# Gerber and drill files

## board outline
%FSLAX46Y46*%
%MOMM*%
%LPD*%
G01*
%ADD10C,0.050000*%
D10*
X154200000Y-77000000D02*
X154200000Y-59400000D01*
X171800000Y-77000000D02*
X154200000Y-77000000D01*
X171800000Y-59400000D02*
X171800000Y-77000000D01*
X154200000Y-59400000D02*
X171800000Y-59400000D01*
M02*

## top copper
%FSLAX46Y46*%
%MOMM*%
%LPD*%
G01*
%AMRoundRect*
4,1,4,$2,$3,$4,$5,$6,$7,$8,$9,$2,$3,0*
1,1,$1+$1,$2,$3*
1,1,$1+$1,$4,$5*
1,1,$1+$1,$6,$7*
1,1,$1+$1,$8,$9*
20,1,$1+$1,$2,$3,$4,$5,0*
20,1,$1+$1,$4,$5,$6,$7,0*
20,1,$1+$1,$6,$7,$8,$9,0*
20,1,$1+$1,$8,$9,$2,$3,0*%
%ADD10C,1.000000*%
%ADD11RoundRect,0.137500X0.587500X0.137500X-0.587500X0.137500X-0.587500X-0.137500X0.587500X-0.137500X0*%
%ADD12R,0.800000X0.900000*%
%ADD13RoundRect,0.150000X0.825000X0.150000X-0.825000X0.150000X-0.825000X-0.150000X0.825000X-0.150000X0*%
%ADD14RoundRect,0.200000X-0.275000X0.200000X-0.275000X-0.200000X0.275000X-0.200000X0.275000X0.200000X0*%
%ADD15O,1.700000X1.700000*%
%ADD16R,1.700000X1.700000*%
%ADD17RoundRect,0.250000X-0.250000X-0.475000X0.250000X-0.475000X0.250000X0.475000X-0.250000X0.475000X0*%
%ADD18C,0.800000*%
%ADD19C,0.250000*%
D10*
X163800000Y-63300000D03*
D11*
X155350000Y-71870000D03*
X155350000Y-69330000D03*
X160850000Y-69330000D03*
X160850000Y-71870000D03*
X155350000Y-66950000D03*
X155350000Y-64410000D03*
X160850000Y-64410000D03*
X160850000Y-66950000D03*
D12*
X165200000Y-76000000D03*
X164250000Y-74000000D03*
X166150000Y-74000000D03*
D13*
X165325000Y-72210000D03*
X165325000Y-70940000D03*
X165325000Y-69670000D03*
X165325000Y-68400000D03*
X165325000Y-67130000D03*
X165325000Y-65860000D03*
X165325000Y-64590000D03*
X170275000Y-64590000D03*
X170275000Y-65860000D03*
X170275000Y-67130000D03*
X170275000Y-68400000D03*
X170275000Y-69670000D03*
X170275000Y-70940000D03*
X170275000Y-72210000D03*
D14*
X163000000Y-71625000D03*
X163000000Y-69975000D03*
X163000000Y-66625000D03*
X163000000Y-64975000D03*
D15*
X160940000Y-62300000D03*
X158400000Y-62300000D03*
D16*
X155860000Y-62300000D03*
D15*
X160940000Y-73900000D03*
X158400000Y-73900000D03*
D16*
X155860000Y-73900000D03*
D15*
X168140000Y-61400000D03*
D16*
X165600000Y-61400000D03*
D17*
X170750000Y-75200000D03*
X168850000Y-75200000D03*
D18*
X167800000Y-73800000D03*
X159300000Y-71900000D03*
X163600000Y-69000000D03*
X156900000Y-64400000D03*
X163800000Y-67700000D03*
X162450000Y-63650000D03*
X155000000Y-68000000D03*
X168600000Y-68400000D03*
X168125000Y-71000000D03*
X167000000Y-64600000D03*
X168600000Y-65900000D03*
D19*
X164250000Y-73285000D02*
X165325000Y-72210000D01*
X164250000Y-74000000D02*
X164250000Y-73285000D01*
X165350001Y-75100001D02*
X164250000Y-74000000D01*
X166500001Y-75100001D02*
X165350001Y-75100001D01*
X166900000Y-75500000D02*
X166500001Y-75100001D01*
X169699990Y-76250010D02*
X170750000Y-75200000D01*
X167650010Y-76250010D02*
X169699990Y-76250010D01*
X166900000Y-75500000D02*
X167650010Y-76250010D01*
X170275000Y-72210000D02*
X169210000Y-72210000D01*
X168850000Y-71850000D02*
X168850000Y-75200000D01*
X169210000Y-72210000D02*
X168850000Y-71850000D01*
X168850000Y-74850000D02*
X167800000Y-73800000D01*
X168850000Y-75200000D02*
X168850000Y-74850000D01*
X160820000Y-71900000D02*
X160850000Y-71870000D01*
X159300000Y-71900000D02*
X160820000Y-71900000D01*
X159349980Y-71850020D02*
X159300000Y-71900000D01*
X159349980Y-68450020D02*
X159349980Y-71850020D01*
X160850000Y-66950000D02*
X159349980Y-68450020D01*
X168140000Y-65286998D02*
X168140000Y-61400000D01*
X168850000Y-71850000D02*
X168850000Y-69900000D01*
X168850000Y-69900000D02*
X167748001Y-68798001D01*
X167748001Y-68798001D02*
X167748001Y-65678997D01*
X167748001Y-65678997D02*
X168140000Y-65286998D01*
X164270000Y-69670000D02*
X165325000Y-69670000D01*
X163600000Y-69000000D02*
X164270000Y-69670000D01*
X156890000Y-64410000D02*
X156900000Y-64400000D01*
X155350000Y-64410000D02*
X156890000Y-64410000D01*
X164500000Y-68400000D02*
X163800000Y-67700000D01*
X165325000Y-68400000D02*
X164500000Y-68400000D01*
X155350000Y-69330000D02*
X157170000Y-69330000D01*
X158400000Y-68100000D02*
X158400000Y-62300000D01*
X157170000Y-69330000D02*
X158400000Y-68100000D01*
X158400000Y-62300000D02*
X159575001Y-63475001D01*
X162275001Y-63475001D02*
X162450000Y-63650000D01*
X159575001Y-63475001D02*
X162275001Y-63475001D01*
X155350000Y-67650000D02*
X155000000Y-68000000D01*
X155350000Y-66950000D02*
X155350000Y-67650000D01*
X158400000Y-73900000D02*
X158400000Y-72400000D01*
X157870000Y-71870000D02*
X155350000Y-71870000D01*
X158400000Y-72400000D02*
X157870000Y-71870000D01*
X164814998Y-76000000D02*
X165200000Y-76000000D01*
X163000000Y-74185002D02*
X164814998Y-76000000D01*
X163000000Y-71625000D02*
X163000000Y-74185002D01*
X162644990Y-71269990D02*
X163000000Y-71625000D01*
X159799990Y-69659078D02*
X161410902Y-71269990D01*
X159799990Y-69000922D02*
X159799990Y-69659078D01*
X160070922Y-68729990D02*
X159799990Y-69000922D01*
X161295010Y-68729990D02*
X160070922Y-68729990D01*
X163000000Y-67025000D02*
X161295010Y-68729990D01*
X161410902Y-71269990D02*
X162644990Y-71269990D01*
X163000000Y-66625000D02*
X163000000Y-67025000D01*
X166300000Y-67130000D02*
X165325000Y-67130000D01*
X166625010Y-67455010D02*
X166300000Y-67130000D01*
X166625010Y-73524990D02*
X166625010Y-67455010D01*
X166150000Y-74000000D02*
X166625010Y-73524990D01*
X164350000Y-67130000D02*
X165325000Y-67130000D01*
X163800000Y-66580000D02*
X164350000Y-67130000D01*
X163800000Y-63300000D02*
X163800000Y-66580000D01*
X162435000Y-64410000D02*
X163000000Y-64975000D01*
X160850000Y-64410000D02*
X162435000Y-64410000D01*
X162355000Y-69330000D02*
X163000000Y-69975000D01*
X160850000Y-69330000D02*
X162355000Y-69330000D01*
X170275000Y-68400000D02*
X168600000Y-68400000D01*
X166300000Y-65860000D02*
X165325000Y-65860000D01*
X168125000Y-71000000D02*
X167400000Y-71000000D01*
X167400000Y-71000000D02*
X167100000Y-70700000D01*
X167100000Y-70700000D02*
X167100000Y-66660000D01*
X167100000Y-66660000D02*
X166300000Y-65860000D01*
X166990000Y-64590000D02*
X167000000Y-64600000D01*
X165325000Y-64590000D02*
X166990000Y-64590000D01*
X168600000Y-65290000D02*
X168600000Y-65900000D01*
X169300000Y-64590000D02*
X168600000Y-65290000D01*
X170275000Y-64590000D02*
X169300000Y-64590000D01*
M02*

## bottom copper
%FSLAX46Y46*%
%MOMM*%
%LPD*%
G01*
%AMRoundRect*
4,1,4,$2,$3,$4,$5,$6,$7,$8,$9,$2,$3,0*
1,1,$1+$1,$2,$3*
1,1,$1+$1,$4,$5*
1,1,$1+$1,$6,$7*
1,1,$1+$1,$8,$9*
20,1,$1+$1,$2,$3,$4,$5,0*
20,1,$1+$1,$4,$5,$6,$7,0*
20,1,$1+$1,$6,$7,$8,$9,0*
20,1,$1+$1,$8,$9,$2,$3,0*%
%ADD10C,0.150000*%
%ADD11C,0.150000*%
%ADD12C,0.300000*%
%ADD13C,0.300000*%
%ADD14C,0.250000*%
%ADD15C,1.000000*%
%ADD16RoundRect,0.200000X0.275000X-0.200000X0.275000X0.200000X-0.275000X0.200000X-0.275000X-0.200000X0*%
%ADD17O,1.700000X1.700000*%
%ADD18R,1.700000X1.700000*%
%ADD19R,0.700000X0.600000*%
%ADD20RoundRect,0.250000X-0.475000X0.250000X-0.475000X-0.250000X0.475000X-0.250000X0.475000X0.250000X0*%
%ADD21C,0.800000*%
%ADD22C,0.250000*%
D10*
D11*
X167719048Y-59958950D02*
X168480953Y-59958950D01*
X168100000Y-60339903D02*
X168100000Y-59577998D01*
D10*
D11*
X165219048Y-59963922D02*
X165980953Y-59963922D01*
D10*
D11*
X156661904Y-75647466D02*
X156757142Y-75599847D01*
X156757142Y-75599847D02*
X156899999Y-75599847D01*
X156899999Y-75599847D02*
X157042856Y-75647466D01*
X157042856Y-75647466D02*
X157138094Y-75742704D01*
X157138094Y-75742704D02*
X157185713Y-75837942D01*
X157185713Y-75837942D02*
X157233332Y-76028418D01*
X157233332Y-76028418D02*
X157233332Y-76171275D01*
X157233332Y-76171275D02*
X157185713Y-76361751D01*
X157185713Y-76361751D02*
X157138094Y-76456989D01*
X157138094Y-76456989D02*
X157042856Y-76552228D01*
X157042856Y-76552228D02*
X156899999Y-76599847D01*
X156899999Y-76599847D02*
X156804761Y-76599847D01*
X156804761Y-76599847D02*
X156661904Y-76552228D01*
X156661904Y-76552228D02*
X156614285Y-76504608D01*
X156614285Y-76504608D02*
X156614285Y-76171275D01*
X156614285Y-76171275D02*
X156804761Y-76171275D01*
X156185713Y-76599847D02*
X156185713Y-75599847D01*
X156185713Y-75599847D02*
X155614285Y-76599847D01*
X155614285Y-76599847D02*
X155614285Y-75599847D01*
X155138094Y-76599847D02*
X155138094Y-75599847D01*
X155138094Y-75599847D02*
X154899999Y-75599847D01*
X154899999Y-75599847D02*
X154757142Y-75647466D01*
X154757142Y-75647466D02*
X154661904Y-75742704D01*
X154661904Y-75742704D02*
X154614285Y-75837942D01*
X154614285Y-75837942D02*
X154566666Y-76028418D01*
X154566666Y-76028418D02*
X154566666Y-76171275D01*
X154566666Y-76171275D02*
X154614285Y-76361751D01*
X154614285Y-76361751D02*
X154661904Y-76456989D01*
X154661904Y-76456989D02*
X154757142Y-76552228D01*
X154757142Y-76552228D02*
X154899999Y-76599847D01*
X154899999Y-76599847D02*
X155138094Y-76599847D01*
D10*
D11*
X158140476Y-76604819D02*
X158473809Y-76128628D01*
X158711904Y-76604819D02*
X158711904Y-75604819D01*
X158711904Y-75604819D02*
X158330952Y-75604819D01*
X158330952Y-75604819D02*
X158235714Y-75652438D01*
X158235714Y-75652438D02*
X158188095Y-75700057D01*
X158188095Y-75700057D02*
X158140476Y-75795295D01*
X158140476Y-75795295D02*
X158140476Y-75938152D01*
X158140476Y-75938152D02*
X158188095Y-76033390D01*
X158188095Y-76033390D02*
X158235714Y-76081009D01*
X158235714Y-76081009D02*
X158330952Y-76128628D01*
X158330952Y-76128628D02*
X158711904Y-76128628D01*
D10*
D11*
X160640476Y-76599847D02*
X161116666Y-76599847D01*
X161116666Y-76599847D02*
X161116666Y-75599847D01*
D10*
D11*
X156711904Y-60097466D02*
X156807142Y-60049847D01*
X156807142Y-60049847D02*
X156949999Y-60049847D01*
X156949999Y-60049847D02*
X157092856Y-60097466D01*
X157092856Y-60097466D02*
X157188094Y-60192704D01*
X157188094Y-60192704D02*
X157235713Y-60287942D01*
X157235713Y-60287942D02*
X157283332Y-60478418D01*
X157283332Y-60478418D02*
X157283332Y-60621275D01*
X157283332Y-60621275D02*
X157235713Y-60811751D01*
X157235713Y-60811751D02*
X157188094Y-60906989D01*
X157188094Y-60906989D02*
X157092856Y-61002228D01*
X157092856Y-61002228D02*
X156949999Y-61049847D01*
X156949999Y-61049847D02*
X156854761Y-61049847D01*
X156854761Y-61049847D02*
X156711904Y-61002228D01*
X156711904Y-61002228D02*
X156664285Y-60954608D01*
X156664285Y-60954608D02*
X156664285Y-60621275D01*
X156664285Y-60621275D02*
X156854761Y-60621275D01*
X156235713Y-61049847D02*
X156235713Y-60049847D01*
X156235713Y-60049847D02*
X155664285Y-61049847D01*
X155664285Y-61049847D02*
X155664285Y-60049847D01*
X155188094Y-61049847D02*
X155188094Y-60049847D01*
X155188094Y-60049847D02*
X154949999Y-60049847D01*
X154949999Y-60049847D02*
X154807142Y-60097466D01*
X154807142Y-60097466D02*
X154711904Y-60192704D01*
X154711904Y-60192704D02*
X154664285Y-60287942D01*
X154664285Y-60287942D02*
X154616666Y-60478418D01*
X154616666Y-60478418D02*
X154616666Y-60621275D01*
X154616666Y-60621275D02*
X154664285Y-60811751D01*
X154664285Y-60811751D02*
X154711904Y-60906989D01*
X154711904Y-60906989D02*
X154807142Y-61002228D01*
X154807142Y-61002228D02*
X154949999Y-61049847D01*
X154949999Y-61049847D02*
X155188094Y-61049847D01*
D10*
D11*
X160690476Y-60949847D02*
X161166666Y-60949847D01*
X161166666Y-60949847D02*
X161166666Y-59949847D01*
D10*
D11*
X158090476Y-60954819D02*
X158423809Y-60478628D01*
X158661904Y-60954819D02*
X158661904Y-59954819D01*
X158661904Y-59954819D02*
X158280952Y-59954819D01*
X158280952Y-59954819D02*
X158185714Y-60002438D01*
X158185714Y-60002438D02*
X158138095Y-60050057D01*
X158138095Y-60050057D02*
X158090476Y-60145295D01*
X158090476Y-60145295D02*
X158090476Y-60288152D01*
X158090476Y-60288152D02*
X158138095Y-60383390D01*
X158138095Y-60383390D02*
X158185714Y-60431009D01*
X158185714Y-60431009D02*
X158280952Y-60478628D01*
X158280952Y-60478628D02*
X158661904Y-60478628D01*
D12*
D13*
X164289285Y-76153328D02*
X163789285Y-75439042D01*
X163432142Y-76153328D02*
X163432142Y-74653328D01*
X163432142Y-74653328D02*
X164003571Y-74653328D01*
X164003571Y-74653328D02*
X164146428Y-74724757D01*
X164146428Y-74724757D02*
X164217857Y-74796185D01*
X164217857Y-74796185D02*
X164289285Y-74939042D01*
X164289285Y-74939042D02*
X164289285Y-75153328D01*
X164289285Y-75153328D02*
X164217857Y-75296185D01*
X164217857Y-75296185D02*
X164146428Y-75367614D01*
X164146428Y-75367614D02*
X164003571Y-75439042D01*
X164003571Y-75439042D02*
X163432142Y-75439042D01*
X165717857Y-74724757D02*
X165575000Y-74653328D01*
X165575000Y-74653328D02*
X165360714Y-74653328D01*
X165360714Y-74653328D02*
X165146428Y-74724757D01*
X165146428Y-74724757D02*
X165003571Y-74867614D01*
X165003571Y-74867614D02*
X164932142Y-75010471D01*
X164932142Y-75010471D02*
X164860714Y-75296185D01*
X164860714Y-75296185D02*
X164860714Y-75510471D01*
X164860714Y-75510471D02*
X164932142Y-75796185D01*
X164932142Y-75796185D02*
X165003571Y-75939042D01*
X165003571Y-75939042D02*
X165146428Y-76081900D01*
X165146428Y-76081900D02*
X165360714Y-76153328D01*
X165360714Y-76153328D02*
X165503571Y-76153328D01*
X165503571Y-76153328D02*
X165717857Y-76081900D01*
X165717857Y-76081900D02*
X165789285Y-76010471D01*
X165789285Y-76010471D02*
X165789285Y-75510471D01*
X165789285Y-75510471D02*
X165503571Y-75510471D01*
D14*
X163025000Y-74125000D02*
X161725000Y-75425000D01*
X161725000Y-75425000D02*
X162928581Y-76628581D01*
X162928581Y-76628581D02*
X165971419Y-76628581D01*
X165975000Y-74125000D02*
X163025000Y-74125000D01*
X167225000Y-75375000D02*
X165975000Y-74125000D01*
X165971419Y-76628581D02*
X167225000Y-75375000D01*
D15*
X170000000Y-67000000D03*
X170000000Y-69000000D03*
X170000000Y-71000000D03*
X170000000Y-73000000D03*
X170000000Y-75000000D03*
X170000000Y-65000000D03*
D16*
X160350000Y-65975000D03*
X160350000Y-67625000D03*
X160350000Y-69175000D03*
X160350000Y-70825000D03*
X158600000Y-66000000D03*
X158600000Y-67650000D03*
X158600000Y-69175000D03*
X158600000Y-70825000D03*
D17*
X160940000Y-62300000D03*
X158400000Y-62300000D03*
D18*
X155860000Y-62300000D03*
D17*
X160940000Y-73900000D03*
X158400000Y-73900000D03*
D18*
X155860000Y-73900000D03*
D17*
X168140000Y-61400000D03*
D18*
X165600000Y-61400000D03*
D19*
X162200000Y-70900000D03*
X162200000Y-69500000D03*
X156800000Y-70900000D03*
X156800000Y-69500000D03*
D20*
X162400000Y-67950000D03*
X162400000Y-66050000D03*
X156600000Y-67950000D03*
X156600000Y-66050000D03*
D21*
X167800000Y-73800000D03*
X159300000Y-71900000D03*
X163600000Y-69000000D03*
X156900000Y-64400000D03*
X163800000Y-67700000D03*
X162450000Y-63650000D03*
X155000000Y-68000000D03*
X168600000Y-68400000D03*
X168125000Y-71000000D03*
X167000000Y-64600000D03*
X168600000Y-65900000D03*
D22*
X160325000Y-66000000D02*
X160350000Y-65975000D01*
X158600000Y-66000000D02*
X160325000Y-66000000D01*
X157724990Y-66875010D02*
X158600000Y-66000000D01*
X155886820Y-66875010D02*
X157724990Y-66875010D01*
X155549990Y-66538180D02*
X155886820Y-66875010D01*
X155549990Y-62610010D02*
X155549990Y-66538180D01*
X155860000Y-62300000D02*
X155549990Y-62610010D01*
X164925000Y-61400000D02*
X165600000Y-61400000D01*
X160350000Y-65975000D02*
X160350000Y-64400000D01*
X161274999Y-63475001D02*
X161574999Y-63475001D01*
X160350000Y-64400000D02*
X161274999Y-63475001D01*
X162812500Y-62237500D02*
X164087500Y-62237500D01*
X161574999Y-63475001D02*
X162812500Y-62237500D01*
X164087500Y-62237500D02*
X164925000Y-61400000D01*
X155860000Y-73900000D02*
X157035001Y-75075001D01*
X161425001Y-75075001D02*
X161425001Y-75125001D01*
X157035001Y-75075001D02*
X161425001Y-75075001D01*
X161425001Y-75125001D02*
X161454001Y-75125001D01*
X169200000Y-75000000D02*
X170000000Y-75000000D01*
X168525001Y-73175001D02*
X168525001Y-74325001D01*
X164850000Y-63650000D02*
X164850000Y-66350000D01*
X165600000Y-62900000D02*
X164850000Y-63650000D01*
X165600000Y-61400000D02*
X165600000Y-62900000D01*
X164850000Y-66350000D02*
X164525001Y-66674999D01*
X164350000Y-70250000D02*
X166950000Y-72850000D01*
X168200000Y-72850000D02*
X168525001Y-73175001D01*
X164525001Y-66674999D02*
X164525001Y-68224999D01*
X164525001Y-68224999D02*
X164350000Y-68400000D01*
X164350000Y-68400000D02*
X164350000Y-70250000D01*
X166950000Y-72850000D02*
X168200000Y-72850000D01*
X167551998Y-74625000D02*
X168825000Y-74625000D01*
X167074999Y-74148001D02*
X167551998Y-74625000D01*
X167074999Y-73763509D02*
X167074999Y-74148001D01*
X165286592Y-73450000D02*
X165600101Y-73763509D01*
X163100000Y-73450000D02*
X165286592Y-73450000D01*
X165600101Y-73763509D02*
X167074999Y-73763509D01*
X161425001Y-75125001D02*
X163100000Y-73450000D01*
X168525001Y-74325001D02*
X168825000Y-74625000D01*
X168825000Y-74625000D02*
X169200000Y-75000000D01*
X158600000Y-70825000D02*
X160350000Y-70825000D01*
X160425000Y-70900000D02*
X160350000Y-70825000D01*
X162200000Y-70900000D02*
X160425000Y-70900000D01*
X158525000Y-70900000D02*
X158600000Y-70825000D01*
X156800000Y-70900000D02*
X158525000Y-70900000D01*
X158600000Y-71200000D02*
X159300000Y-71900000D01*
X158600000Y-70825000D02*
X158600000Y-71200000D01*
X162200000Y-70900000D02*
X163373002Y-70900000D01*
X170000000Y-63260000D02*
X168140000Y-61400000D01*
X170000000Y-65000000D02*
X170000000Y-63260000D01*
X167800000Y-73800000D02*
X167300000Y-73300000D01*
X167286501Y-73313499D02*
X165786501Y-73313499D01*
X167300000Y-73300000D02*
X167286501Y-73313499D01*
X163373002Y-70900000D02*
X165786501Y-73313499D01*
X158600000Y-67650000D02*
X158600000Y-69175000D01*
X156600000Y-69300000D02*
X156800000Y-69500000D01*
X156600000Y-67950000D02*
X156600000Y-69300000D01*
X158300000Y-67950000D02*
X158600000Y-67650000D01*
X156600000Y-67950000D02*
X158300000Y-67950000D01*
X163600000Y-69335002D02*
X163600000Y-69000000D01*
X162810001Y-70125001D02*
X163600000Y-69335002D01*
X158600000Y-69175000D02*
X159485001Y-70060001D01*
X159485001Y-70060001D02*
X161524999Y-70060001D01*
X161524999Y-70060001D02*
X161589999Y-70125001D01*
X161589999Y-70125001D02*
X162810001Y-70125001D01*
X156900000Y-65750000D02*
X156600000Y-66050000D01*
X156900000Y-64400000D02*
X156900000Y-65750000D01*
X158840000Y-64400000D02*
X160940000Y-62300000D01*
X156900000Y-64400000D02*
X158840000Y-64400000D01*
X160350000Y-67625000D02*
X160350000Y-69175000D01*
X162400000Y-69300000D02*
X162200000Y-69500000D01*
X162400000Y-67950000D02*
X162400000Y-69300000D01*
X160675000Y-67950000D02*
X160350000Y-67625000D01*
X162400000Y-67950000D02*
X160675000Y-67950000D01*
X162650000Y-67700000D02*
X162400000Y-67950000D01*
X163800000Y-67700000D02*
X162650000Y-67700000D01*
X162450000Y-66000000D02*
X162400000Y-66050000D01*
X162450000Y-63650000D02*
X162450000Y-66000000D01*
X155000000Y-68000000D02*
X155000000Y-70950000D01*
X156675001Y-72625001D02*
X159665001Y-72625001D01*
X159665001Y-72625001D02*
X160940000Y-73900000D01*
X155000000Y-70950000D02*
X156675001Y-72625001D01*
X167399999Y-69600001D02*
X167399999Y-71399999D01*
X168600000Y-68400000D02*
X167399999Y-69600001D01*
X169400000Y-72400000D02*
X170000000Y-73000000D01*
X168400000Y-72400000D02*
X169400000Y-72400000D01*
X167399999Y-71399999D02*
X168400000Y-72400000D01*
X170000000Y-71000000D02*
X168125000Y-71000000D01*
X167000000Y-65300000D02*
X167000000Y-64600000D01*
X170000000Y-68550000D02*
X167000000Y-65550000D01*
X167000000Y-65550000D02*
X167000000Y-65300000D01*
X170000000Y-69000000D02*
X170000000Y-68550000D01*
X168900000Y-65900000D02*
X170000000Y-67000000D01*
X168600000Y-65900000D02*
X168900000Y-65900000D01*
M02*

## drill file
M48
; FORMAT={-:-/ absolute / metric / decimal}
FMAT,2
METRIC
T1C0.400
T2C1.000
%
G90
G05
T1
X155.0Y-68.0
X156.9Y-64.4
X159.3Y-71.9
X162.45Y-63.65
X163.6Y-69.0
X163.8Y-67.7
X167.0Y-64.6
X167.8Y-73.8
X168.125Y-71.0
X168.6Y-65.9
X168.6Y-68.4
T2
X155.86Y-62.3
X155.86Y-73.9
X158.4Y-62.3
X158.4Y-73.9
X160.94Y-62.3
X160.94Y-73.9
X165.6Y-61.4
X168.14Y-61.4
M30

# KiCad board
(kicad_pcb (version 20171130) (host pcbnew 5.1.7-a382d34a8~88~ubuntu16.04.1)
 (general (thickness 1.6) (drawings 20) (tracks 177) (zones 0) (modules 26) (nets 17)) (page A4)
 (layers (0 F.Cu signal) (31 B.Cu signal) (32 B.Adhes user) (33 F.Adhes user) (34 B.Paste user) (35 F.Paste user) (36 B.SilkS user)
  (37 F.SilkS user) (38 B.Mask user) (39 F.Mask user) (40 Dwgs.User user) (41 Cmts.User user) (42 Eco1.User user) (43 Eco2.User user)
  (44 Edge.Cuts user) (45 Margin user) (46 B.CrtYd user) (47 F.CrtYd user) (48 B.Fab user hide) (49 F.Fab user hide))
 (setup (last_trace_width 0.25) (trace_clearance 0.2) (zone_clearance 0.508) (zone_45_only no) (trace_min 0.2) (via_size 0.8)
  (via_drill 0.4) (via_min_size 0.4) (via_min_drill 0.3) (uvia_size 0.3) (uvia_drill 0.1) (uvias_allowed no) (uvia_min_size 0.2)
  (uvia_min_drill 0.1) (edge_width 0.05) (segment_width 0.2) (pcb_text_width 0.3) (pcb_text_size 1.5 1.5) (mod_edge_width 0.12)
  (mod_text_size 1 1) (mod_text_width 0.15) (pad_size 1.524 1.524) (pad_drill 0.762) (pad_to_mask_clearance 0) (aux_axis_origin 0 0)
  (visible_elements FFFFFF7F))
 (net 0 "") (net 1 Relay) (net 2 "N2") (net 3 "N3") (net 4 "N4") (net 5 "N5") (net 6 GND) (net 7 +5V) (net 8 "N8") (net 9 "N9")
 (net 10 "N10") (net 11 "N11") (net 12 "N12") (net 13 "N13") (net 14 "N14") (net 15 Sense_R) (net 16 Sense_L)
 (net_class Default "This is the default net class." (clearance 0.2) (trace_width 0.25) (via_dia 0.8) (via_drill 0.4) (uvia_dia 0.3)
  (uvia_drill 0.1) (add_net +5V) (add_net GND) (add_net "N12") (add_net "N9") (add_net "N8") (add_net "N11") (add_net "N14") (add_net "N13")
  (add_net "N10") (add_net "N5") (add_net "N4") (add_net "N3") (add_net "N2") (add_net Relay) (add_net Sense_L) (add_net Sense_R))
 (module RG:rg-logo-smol (layer F.Cu) (at 164.55 75.4)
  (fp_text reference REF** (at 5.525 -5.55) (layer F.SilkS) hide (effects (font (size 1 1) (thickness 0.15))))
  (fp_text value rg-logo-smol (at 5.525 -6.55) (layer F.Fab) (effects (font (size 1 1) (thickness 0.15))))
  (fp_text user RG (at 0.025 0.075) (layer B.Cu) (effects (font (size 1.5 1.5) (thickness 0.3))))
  (fp_line (start -1.525 -1.275) (end -2.825 0.025) (layer B.Cu) (width 0.25))
  (fp_line (start -2.825 0.025) (end -1.621419 1.228581) (layer B.Cu) (width 0.25))
  (fp_line (start -1.621419 1.228581) (end 1.421419 1.228581) (layer B.Cu) (width 0.25))
  (fp_line (start 1.425 -1.275) (end -1.525 -1.275) (layer B.Cu) (width 0.25))
  (fp_line (start 2.675 -0.025) (end 1.425 -1.275) (layer B.Cu) (width 0.25))
  (fp_line (start 1.421419 1.228581) (end 2.675 -0.025) (layer B.Cu) (width 0.25)))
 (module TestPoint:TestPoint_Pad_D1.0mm (layer F.Cu) (at 163.8 63.3)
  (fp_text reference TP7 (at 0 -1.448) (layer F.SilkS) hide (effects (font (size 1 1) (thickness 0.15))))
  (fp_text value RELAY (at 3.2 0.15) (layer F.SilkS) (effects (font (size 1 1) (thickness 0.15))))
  (pad 1 smd circle (at 0 0) (size 1 1) (layers F.Cu F.Mask) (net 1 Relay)))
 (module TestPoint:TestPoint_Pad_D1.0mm (layer B.Cu) (at 170 67)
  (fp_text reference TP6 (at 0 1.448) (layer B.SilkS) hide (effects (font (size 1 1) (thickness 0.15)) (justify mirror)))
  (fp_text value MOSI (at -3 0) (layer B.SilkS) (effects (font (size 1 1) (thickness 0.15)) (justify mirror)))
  (pad 1 smd circle (at 0 0) (size 1 1) (layers B.Cu B.Mask) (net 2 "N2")))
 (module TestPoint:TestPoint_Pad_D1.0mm (layer B.Cu) (at 170 69)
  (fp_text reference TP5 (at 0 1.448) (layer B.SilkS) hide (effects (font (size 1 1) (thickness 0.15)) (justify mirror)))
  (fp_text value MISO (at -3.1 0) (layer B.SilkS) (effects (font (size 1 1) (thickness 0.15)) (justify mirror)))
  (pad 1 smd circle (at 0 0) (size 1 1) (layers B.Cu B.Mask) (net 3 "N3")))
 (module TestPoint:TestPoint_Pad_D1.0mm (layer B.Cu) (at 170 71)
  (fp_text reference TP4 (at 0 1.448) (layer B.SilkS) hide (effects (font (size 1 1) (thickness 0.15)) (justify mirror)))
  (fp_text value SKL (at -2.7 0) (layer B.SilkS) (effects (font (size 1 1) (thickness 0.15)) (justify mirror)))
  (pad 1 smd circle (at 0 0) (size 1 1) (layers B.Cu B.Mask) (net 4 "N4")))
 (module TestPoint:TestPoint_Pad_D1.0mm (layer B.Cu) (at 170 73)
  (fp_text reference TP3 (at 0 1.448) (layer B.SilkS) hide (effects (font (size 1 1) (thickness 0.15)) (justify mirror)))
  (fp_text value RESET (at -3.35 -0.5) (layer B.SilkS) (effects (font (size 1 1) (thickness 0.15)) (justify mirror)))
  (pad 1 smd circle (at 0 0) (size 1 1) (layers B.Cu B.Mask) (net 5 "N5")))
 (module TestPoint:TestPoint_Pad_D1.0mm (layer B.Cu) (at 170 75)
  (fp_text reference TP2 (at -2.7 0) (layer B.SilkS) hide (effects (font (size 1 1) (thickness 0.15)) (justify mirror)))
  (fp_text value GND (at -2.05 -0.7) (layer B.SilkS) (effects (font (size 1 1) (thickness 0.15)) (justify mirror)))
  (pad 1 smd circle (at 0 0) (size 1 1) (layers B.Cu B.Mask) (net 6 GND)))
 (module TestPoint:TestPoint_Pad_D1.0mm (layer B.Cu) (at 170 65)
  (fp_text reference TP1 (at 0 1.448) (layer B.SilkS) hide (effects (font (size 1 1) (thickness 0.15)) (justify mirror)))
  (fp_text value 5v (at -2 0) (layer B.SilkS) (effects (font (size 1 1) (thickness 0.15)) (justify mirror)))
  (pad 1 smd circle (at 0 0) (size 1 1) (layers B.Cu B.Mask) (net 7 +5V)))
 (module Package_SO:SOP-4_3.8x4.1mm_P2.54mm (layer F.Cu) (at 158.1 70.6 180)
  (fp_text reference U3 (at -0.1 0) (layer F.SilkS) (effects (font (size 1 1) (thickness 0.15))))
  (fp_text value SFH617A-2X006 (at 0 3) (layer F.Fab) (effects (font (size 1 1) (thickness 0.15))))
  (pad 4 smd roundrect (at 2.75 -1.27 180) (size 1.45 0.55) (layers F.Cu F.Paste F.Mask) (roundrect_rratio 0.25) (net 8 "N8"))
  (pad 3 smd roundrect (at 2.75 1.27 180) (size 1.45 0.55) (layers F.Cu F.Paste F.Mask) (roundrect_rratio 0.25) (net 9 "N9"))
  (pad 2 smd roundrect (at -2.75 1.27 180) (size 1.45 0.55) (layers F.Cu F.Paste F.Mask) (roundrect_rratio 0.25) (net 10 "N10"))
  (pad 1 smd roundrect (at -2.75 -1.27 180) (size 1.45 0.55) (layers F.Cu F.Paste F.Mask) (roundrect_rratio 0.25) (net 7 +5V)))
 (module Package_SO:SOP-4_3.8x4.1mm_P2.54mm (layer F.Cu) (at 158.1 65.68 180)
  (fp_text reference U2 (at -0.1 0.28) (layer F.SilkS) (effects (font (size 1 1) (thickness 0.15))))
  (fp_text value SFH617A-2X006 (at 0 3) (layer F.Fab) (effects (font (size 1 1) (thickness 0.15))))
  (pad 4 smd roundrect (at 2.75 -1.27 180) (size 1.45 0.55) (layers F.Cu F.Paste F.Mask) (roundrect_rratio 0.25) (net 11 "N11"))
  (pad 3 smd roundrect (at 2.75 1.27 180) (size 1.45 0.55) (layers F.Cu F.Paste F.Mask) (roundrect_rratio 0.25) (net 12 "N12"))
  (pad 2 smd roundrect (at -2.75 1.27 180) (size 1.45 0.55) (layers F.Cu F.Paste F.Mask) (roundrect_rratio 0.25) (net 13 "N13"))
  (pad 1 smd roundrect (at -2.75 -1.27 180) (size 1.45 0.55) (layers F.Cu F.Paste F.Mask) (roundrect_rratio 0.25) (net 7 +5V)))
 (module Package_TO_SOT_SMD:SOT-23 (layer F.Cu) (at 165.2 75 270)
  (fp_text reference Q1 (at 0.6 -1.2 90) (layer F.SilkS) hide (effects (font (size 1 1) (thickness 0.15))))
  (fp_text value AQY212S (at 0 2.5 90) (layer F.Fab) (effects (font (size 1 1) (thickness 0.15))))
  (pad 3 smd rect (at 1 0 270) (size 0.9 0.8) (layers F.Cu F.Paste F.Mask) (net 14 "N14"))
  (pad 2 smd rect (at -1 0.95 270) (size 0.9 0.8) (layers F.Cu F.Paste F.Mask) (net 6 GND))
  (pad 1 smd rect (at -1 -0.95 270) (size 0.9 0.8) (layers F.Cu F.Paste F.Mask) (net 1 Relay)))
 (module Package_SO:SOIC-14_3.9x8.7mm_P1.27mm (layer F.Cu) (at 167.8 68.4 180)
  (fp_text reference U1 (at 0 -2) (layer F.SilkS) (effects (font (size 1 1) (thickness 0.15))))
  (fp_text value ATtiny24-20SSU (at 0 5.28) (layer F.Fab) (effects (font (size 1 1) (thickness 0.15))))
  (pad 14 smd roundrect (at 2.475 -3.81 180) (size 1.95 0.6) (layers F.Cu F.Paste F.Mask) (roundrect_rratio 0.25) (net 6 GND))
  (pad 13 smd roundrect (at 2.475 -2.54 180) (size 1.95 0.6) (layers F.Cu F.Paste F.Mask) (roundrect_rratio 0.25))
  (pad 12 smd roundrect (at 2.475 -1.27 180) (size 1.95 0.6) (layers F.Cu F.Paste F.Mask) (roundrect_rratio 0.25) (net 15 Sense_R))
  (pad 11 smd roundrect (at 2.475 0 180) (size 1.95 0.6) (layers F.Cu F.Paste F.Mask) (roundrect_rratio 0.25) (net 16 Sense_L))
  (pad 10 smd roundrect (at 2.475 1.27 180) (size 1.95 0.6) (layers F.Cu F.Paste F.Mask) (roundrect_rratio 0.25) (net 1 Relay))
  (pad 9 smd roundrect (at 2.475 2.54 180) (size 1.95 0.6) (layers F.Cu F.Paste F.Mask) (roundrect_rratio 0.25) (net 4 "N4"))
  (pad 8 smd roundrect (at 2.475 3.81 180) (size 1.95 0.6) (layers F.Cu F.Paste F.Mask) (roundrect_rratio 0.25) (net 3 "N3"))
  (pad 7 smd roundrect (at -2.475 3.81 180) (size 1.95 0.6) (layers F.Cu F.Paste F.Mask) (roundrect_rratio 0.25) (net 2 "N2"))
  (pad 6 smd roundrect (at -2.475 2.54 180) (size 1.95 0.6) (layers F.Cu F.Paste F.Mask) (roundrect_rratio 0.25))
  (pad 5 smd roundrect (at -2.475 1.27 180) (size 1.95 0.6) (layers F.Cu F.Paste F.Mask) (roundrect_rratio 0.25))
  (pad 4 smd roundrect (at -2.475 0 180) (size 1.95 0.6) (layers F.Cu F.Paste F.Mask) (roundrect_rratio 0.25) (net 5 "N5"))
  (pad 3 smd roundrect (at -2.475 -1.27 180) (size 1.95 0.6) (layers F.Cu F.Paste F.Mask) (roundrect_rratio 0.25))
  (pad 2 smd roundrect (at -2.475 -2.54 180) (size 1.95 0.6) (layers F.Cu F.Paste F.Mask) (roundrect_rratio 0.25))
  (pad 1 smd roundrect (at -2.475 -3.81 180) (size 1.95 0.6) (layers F.Cu F.Paste F.Mask) (roundrect_rratio 0.25) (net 7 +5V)))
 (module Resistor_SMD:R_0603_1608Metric (layer F.Cu) (at 163 70.8 270)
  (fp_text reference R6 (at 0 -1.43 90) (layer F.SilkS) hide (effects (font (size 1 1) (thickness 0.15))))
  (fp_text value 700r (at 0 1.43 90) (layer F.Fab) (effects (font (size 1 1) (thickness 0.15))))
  (pad 2 smd roundrect (at 0.825 0 270) (size 0.8 0.95) (layers F.Cu F.Paste F.Mask) (roundrect_rratio 0.25) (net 14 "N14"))
  (pad 1 smd roundrect (at -0.825 0 270) (size 0.8 0.95) (layers F.Cu F.Paste F.Mask) (roundrect_rratio 0.25) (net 10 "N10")))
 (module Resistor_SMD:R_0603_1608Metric (layer F.Cu) (at 163 65.8 270)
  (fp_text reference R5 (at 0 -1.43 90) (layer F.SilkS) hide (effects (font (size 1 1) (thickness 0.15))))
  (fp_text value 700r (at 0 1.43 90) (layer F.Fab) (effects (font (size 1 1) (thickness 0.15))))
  (pad 2 smd roundrect (at 0.825 0 270) (size 0.8 0.95) (layers F.Cu F.Paste F.Mask) (roundrect_rratio 0.25) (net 14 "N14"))
  (pad 1 smd roundrect (at -0.825 0 270) (size 0.8 0.95) (layers F.Cu F.Paste F.Mask) (roundrect_rratio 0.25) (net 13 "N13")))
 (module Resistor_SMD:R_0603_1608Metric (layer B.Cu) (at 160.35 66.8 90)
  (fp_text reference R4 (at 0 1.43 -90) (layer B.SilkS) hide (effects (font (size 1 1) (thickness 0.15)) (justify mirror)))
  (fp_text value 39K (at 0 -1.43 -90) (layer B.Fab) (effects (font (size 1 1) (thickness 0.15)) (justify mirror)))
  (pad 2 smd roundrect (at 0.825 0 90) (size 0.8 0.95) (layers B.Cu B.Paste B.Mask) (roundrect_rratio 0.25) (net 6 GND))
  (pad 1 smd roundrect (at -0.825 0 90) (size 0.8 0.95) (layers B.Cu B.Paste B.Mask) (roundrect_rratio 0.25) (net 16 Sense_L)))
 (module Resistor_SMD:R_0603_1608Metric (layer B.Cu) (at 160.35 70 90)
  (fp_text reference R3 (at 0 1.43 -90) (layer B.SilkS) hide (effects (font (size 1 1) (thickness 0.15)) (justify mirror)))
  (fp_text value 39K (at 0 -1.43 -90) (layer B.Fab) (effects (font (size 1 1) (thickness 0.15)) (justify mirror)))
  (pad 2 smd roundrect (at 0.825 0 90) (size 0.8 0.95) (layers B.Cu B.Paste B.Mask) (roundrect_rratio 0.25) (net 16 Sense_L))
  (pad 1 smd roundrect (at -0.825 0 90) (size 0.8 0.95) (layers B.Cu B.Paste B.Mask) (roundrect_rratio 0.25) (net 7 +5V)))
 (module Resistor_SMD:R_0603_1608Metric (layer B.Cu) (at 158.6 66.825 90)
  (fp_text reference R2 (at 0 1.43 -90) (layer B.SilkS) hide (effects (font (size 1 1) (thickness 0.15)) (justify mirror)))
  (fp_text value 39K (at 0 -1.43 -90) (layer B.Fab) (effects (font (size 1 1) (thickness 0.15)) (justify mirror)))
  (pad 2 smd roundrect (at 0.825 0 90) (size 0.8 0.95) (layers B.Cu B.Paste B.Mask) (roundrect_rratio 0.25) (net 6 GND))
  (pad 1 smd roundrect (at -0.825 0 90) (size 0.8 0.95) (layers B.Cu B.Paste B.Mask) (roundrect_rratio 0.25) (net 15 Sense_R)))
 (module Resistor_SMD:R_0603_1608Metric (layer B.Cu) (at 158.6 70 90)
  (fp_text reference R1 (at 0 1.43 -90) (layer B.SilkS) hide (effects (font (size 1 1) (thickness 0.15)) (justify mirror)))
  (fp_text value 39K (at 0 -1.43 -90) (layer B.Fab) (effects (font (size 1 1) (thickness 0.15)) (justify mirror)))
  (pad 2 smd roundrect (at 0.825 0 90) (size 0.8 0.95) (layers B.Cu B.Paste B.Mask) (roundrect_rratio 0.25) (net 15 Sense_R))
  (pad 1 smd roundrect (at -0.825 0 90) (size 0.8 0.95) (layers B.Cu B.Paste B.Mask) (roundrect_rratio 0.25) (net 7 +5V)))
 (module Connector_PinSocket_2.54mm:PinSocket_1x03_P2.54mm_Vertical (layer F.Cu) (at 155.86 62.3 90)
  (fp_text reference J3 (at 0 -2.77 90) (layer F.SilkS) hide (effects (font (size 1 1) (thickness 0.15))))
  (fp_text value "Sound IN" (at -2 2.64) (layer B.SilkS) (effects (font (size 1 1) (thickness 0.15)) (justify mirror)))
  (pad 3 thru_hole oval (at 0 5.08 90) (size 1.7 1.7) (drill 1) (layers *.Cu *.Mask) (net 12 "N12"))
  (pad 2 thru_hole oval (at 0 2.54 90) (size 1.7 1.7) (drill 1) (layers *.Cu *.Mask) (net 9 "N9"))
  (pad 1 thru_hole rect (at 0 0 90) (size 1.7 1.7) (drill 1) (layers *.Cu *.Mask) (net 6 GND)))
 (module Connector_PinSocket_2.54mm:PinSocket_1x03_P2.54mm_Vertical (layer F.Cu) (at 155.86 73.9 90)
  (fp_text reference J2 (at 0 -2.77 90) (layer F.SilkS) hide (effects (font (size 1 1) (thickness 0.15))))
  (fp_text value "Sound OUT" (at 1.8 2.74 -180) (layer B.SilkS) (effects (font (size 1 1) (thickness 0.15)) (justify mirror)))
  (pad 3 thru_hole oval (at 0 5.08 90) (size 1.7 1.7) (drill 1) (layers *.Cu *.Mask) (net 11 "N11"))
  (pad 2 thru_hole oval (at 0 2.54 90) (size 1.7 1.7) (drill 1) (layers *.Cu *.Mask) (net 8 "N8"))
  (pad 1 thru_hole rect (at 0 0 90) (size 1.7 1.7) (drill 1) (layers *.Cu *.Mask) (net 6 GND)))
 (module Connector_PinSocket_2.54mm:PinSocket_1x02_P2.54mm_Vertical (layer F.Cu) (at 165.6 61.4 90)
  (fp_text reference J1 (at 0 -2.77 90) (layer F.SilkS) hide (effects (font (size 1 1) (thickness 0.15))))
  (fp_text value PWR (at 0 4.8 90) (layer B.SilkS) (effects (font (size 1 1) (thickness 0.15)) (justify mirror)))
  (pad 2 thru_hole oval (at 0 2.54 90) (size 1.7 1.7) (drill 1) (layers *.Cu *.Mask) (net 7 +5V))
  (pad 1 thru_hole rect (at 0 0 90) (size 1.7 1.7) (drill 1) (layers *.Cu *.Mask) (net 6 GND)))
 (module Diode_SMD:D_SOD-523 (layer B.Cu) (at 162.2 70.2 90)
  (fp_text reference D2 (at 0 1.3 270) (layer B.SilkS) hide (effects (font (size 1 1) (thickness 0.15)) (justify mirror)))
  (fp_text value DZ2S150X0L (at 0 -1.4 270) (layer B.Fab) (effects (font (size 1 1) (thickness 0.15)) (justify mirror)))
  (pad 1 smd rect (at -0.7 0 270) (size 0.6 0.7) (layers B.Cu B.Paste B.Mask) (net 7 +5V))
  (pad 2 smd rect (at 0.7 0 270) (size 0.6 0.7) (layers B.Cu B.Paste B.Mask) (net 16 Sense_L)))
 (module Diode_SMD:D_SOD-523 (layer B.Cu) (at 156.8 70.2 90)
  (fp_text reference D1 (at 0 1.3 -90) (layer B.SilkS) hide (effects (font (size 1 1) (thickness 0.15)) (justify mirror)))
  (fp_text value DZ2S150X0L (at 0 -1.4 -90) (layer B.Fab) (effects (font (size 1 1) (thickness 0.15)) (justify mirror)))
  (pad 1 smd rect (at -0.7 0 270) (size 0.6 0.7) (layers B.Cu B.Paste B.Mask) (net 7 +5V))
  (pad 2 smd rect (at 0.7 0 270) (size 0.6 0.7) (layers B.Cu B.Paste B.Mask) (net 15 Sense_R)))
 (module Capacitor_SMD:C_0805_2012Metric (layer B.Cu) (at 162.4 67 270)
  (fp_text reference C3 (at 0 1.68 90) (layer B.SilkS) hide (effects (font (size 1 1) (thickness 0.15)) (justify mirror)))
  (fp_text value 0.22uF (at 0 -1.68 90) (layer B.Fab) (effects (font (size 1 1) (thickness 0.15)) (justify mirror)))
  (pad 2 smd roundrect (at 0.95 0 270) (size 1 1.45) (layers B.Cu B.Paste B.Mask) (roundrect_rratio 0.25) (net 16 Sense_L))
  (pad 1 smd roundrect (at -0.95 0 270) (size 1 1.45) (layers B.Cu B.Paste B.Mask) (roundrect_rratio 0.25) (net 9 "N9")))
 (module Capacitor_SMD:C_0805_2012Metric (layer B.Cu) (at 156.6 67 270)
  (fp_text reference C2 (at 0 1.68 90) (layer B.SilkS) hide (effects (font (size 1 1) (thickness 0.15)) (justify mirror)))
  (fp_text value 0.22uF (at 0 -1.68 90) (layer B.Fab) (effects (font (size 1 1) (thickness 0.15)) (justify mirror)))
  (pad 2 smd roundrect (at 0.95 0 270) (size 1 1.45) (layers B.Cu B.Paste B.Mask) (roundrect_rratio 0.25) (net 15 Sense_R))
  (pad 1 smd roundrect (at -0.95 0 270) (size 1 1.45) (layers B.Cu B.Paste B.Mask) (roundrect_rratio 0.25) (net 12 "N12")))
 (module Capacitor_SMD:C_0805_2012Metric (layer F.Cu) (at 169.8 75.2)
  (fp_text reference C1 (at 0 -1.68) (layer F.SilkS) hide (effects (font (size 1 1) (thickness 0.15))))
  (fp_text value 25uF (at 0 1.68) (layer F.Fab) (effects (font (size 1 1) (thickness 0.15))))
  (pad 2 smd roundrect (at 0.95 0) (size 1 1.45) (layers F.Cu F.Paste F.Mask) (roundrect_rratio 0.25) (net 6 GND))
  (pad 1 smd roundrect (at -0.95 0) (size 1 1.45) (layers F.Cu F.Paste F.Mask) (roundrect_rratio 0.25) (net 7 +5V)))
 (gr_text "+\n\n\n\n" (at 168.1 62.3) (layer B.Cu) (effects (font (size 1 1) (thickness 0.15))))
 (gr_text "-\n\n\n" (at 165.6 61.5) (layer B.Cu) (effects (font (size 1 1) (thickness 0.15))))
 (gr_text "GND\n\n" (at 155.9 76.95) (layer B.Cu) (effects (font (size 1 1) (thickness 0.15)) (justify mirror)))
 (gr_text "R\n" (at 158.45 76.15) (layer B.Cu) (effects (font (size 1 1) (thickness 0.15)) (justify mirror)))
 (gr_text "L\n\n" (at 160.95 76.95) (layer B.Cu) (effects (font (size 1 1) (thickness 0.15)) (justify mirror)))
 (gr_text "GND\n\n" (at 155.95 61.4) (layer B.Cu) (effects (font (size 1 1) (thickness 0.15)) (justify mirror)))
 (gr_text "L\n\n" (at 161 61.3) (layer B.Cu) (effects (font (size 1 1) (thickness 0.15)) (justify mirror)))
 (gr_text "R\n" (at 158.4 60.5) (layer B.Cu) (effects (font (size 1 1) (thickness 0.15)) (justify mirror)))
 (gr_line (start 154.2 77) (end 154.2 59.4) (layer Edge.Cuts) (width 0.05))
 (gr_line (start 171.8 77) (end 154.2 77) (layer Edge.Cuts) (width 0.05))
 (gr_line (start 171.8 59.4) (end 171.8 77) (layer Edge.Cuts) (width 0.05))
 (gr_line (start 154.2 59.4) (end 171.8 59.4) (layer Edge.Cuts) (width 0.05))
 (segment (start 160.325 66) (end 160.35 65.975) (width 0.25) (layer B.Cu) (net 6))
 (segment (start 158.6 66) (end 160.325 66) (width 0.25) (layer B.Cu) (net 6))
 (segment (start 164.25 73.285) (end 165.325 72.21) (width 0.25) (layer F.Cu) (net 6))
 (segment (start 164.25 74) (end 164.25 73.285) (width 0.25) (layer F.Cu) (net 6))
 (segment (start 165.350001 75.100001) (end 164.25 74) (width 0.25) (layer F.Cu) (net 6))
 (segment (start 166.500001 75.100001) (end 165.350001 75.100001) (width 0.25) (layer F.Cu) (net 6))
 (segment (start 166.9 75.5) (end 166.500001 75.100001) (width 0.25) (layer F.Cu) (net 6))
 (segment (start 169.69999 76.25001) (end 170.75 75.2) (width 0.25) (layer F.Cu) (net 6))
 (segment (start 167.65001 76.25001) (end 169.69999 76.25001) (width 0.25) (layer F.Cu) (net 6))
 (segment (start 166.9 75.5) (end 167.65001 76.25001) (width 0.25) (layer F.Cu) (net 6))
 (segment (start 157.72499 66.87501) (end 158.6 66) (width 0.25) (layer B.Cu) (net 6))
 (segment (start 155.88682 66.87501) (end 157.72499 66.87501) (width 0.25) (layer B.Cu) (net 6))
 (segment (start 155.54999 66.53818) (end 155.88682 66.87501) (width 0.25) (layer B.Cu) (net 6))
 (segment (start 155.54999 62.61001) (end 155.54999 66.53818) (width 0.25) (layer B.Cu) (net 6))
 (segment (start 155.86 62.3) (end 155.54999 62.61001) (width 0.25) (layer B.Cu) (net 6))
 (segment (start 164.925 61.4) (end 165.6 61.4) (width 0.25) (layer B.Cu) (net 6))
 (segment (start 160.35 65.975) (end 160.35 64.4) (width 0.25) (layer B.Cu) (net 6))
 (segment (start 161.274999 63.475001) (end 161.574999 63.475001) (width 0.25) (layer B.Cu) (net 6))
 (segment (start 160.35 64.4) (end 161.274999 63.475001) (width 0.25) (layer B.Cu) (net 6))
 (segment (start 162.8125 62.2375) (end 164.0875 62.2375) (width 0.25) (layer B.Cu) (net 6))
 (segment (start 161.574999 63.475001) (end 162.8125 62.2375) (width 0.25) (layer B.Cu) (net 6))
 (segment (start 164.0875 62.2375) (end 164.925 61.4) (width 0.25) (layer B.Cu) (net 6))
 (segment (start 155.86 73.9) (end 157.035001 75.075001) (width 0.25) (layer B.Cu) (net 6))
 (segment (start 161.425001 75.075001) (end 161.425001 75.125001) (width 0.25) (layer B.Cu) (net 6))
 (segment (start 157.035001 75.075001) (end 161.425001 75.075001) (width 0.25) (layer B.Cu) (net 6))
 (segment (start 161.425001 75.125001) (end 161.454001 75.125001) (width 0.25) (layer B.Cu) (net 6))
 (segment (start 169.2 75) (end 170 75) (width 0.25) (layer B.Cu) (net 6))
 (segment (start 168.525001 73.175001) (end 168.525001 74.325001) (width 0.25) (layer B.Cu) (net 6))
 (segment (start 164.85 63.65) (end 164.85 66.35) (width 0.25) (layer B.Cu) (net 6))
 (segment (start 165.6 62.9) (end 164.85 63.65) (width 0.25) (layer B.Cu) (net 6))
 (segment (start 165.6 61.4) (end 165.6 62.9) (width 0.25) (layer B.Cu) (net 6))
 (segment (start 164.85 66.35) (end 164.525001 66.674999) (width 0.25) (layer B.Cu) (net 6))
 (segment (start 164.35 70.25) (end 166.95 72.85) (width 0.25) (layer B.Cu) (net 6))
 (segment (start 168.2 72.85) (end 168.525001 73.175001) (width 0.25) (layer B.Cu) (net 6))
 (segment (start 164.525001 66.674999) (end 164.525001 68.224999) (width 0.25) (layer B.Cu) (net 6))
 (segment (start 164.525001 68.224999) (end 164.35 68.4) (width 0.25) (layer B.Cu) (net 6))
 (segment (start 164.35 68.4) (end 164.35 70.25) (width 0.25) (layer B.Cu) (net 6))
 (segment (start 166.95 72.85) (end 168.2 72.85) (width 0.25) (layer B.Cu) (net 6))
 (segment (start 167.551998 74.625) (end 168.825 74.625) (width 0.25) (layer B.Cu) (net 6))
 (segment (start 167.074999 74.148001) (end 167.551998 74.625) (width 0.25) (layer B.Cu) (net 6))
 (segment (start 167.074999 73.763509) (end 167.074999 74.148001) (width 0.25) (layer B.Cu) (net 6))
 (segment (start 165.286592 73.45) (end 165.600101 73.763509) (width 0.25) (layer B.Cu) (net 6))
 (segment (start 163.1 73.45) (end 165.286592 73.45) (width 0.25) (layer B.Cu) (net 6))
 (segment (start 165.600101 73.763509) (end 167.074999 73.763509) (width 0.25) (layer B.Cu) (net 6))
 (segment (start 161.425001 75.125001) (end 163.1 73.45) (width 0.25) (layer B.Cu) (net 6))
 (segment (start 168.525001 74.325001) (end 168.825 74.625) (width 0.25) (layer B.Cu) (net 6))
 (segment (start 168.825 74.625) (end 169.2 75) (width 0.25) (layer B.Cu) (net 6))
 (segment (start 158.6 70.825) (end 160.35 70.825) (width 0.25) (layer B.Cu) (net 7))
 (segment (start 160.425 70.9) (end 160.35 70.825) (width 0.25) (layer B.Cu) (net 7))
 (segment (start 162.2 70.9) (end 160.425 70.9) (width 0.25) (layer B.Cu) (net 7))
 (segment (start 158.525 70.9) (end 158.6 70.825) (width 0.25) (layer B.Cu) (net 7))
 (segment (start 156.8 70.9) (end 158.525 70.9) (width 0.25) (layer B.Cu) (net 7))
 (segment (start 170.275 72.21) (end 169.21 72.21) (width 0.25) (layer F.Cu) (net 7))
 (segment (start 168.85 71.85) (end 168.85 75.2) (width 0.25) (layer F.Cu) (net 7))
 (segment (start 169.21 72.21) (end 168.85 71.85) (width 0.25) (layer F.Cu) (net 7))
 (via (at 167.8 73.8) (size 0.8) (drill 0.4) (layers F.Cu B.Cu) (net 7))
 (segment (start 168.85 74.85) (end 167.8 73.8) (width 0.25) (layer F.Cu) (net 7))
 (segment (start 168.85 75.2) (end 168.85 74.85) (width 0.25) (layer F.Cu) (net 7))
 (via (at 159.3 71.9) (size 0.8) (drill 0.4) (layers F.Cu B.Cu) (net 7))
 (segment (start 158.6 71.2) (end 159.3 71.9) (width 0.25) (layer B.Cu) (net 7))
 (segment (start 158.6 70.825) (end 158.6 71.2) (width 0.25) (layer B.Cu) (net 7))
 (segment (start 160.82 71.9) (end 160.85 71.87) (width 0.25) (layer F.Cu) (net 7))
 (segment (start 159.3 71.9) (end 160.82 71.9) (width 0.25) (layer F.Cu) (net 7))
 (segment (start 159.34998 71.85002) (end 159.3 71.9) (width 0.25) (layer F.Cu) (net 7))
 (segment (start 159.34998 68.45002) (end 159.34998 71.85002) (width 0.25) (layer F.Cu) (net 7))
 (segment (start 160.85 66.95) (end 159.34998 68.45002) (width 0.25) (layer F.Cu) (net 7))
 (segment (start 162.2 70.9) (end 163.373002 70.9) (width 0.25) (layer B.Cu) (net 7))
 (segment (start 168.14 65.286998) (end 168.14 61.4) (width 0.25) (layer F.Cu) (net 7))
 (segment (start 168.85 71.85) (end 168.85 69.9) (width 0.25) (layer F.Cu) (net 7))
 (segment (start 168.85 69.9) (end 167.748001 68.798001) (width 0.25) (layer F.Cu) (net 7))
 (segment (start 167.748001 68.798001) (end 167.748001 65.678997) (width 0.25) (layer F.Cu) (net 7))
 (segment (start 167.748001 65.678997) (end 168.14 65.286998) (width 0.25) (layer F.Cu) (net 7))
 (segment (start 170 63.26) (end 168.14 61.4) (width 0.25) (layer B.Cu) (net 7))
 (segment (start 170 65) (end 170 63.26) (width 0.25) (layer B.Cu) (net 7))
 (segment (start 167.8 73.8) (end 167.3 73.3) (width 0.25) (layer B.Cu) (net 7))
 (segment (start 167.286501 73.313499) (end 165.786501 73.313499) (width 0.25) (layer B.Cu) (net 7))
 (segment (start 167.3 73.3) (end 167.286501 73.313499) (width 0.25) (layer B.Cu) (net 7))
 (segment (start 163.373002 70.9) (end 165.786501 73.313499) (width 0.25) (layer B.Cu) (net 7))
 (segment (start 158.6 67.65) (end 158.6 69.175) (width 0.25) (layer B.Cu) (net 15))
 (segment (start 156.6 69.3) (end 156.8 69.5) (width 0.25) (layer B.Cu) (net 15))
 (segment (start 156.6 67.95) (end 156.6 69.3) (width 0.25) (layer B.Cu) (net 15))
 (segment (start 158.3 67.95) (end 158.6 67.65) (width 0.25) (layer B.Cu) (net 15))
 (segment (start 156.6 67.95) (end 158.3 67.95) (width 0.25) (layer B.Cu) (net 15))
 (via (at 163.6 69) (size 0.8) (drill 0.4) (layers F.Cu B.Cu) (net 15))
 (segment (start 163.6 69.335002) (end 163.6 69) (width 0.25) (layer B.Cu) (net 15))
 (segment (start 162.810001 70.125001) (end 163.6 69.335002) (width 0.25) (layer B.Cu) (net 15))
 (segment (start 158.6 69.175) (end 159.485001 70.060001) (width 0.25) (layer B.Cu) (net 15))
 (segment (start 159.485001 70.060001) (end 161.524999 70.060001) (width 0.25) (layer B.Cu) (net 15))
 (segment (start 161.524999 70.060001) (end 161.589999 70.125001) (width 0.25) (layer B.Cu) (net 15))
 (segment (start 161.589999 70.125001) (end 162.810001 70.125001) (width 0.25) (layer B.Cu) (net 15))
 (segment (start 164.27 69.67) (end 165.325 69.67) (width 0.25) (layer F.Cu) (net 15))
 (segment (start 163.6 69) (end 164.27 69.67) (width 0.25) (layer F.Cu) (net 15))
 (via (at 156.9 64.4) (size 0.8) (drill 0.4) (layers F.Cu B.Cu) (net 12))
 (segment (start 156.89 64.41) (end 156.9 64.4) (width 0.25) (layer F.Cu) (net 12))
 (segment (start 155.35 64.41) (end 156.89 64.41) (width 0.25) (layer F.Cu) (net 12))
 (segment (start 156.9 65.75) (end 156.6 66.05) (width 0.25) (layer B.Cu) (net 12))
 (segment (start 156.9 64.4) (end 156.9 65.75) (width 0.25) (layer B.Cu) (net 12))
 (segment (start 158.84 64.4) (end 160.94 62.3) (width 0.25) (layer B.Cu) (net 12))
 (segment (start 156.9 64.4) (end 158.84 64.4) (width 0.25) (layer B.Cu) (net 12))
 (segment (start 160.35 67.625) (end 160.35 69.175) (width 0.25) (layer B.Cu) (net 16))
 (segment (start 162.4 69.3) (end 162.2 69.5) (width 0.25) (layer B.Cu) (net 16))
 (segment (start 162.4 67.95) (end 162.4 69.3) (width 0.25) (layer B.Cu) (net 16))
 (segment (start 160.675 67.95) (end 160.35 67.625) (width 0.25) (layer B.Cu) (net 16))
 (segment (start 162.4 67.95) (end 160.675 67.95) (width 0.25) (layer B.Cu) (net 16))
 (segment (start 164.5 68.4) (end 163.8 67.7) (width 0.25) (layer F.Cu) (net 16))
 (via (at 163.8 67.7) (size 0.8) (drill 0.4) (layers F.Cu B.Cu) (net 16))
 (segment (start 165.325 68.4) (end 164.5 68.4) (width 0.25) (layer F.Cu) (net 16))
 (segment (start 162.65 67.7) (end 162.4 67.95) (width 0.25) (layer B.Cu) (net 16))
 (segment (start 163.8 67.7) (end 162.65 67.7) (width 0.25) (layer B.Cu) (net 16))
 (segment (start 155.35 69.33) (end 157.17 69.33) (width 0.25) (layer F.Cu) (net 9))
 (segment (start 158.4 68.1) (end 158.4 62.3) (width 0.25) (layer F.Cu) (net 9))
 (segment (start 157.17 69.33) (end 158.4 68.1) (width 0.25) (layer F.Cu) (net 9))
 (segment (start 158.4 62.3) (end 159.575001 63.475001) (width 0.25) (layer F.Cu) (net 9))
 (via (at 162.45 63.65) (size 0.8) (drill 0.4) (layers F.Cu B.Cu) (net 9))
 (segment (start 162.275001 63.475001) (end 162.45 63.65) (width 0.25) (layer F.Cu) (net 9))
 (segment (start 159.575001 63.475001) (end 162.275001 63.475001) (width 0.25) (layer F.Cu) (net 9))
 (segment (start 162.45 66) (end 162.4 66.05) (width 0.25) (layer B.Cu) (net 9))
 (segment (start 162.45 63.65) (end 162.45 66) (width 0.25) (layer B.Cu) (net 9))
 (via (at 155 68) (size 0.8) (drill 0.4) (layers F.Cu B.Cu) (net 11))
 (segment (start 155.35 67.65) (end 155 68) (width 0.25) (layer F.Cu) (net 11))
 (segment (start 155.35 66.95) (end 155.35 67.65) (width 0.25) (layer F.Cu) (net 11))
 (segment (start 155 68) (end 155 70.95) (width 0.25) (layer B.Cu) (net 11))
 (segment (start 156.675001 72.625001) (end 159.665001 72.625001) (width 0.25) (layer B.Cu) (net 11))
 (segment (start 159.665001 72.625001) (end 160.94 73.9) (width 0.25) (layer B.Cu) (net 11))
 (segment (start 155 70.95) (end 156.675001 72.625001) (width 0.25) (layer B.Cu) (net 11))
 (segment (start 158.4 73.9) (end 158.4 72.4) (width 0.25) (layer F.Cu) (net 8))
 (segment (start 157.87 71.87) (end 155.35 71.87) (width 0.25) (layer F.Cu) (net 8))
 (segment (start 158.4 72.4) (end 157.87 71.87) (width 0.25) (layer F.Cu) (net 8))
 (segment (start 164.814998 76) (end 165.2 76) (width 0.25) (layer F.Cu) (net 14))
 (segment (start 163 74.185002) (end 164.814998 76) (width 0.25) (layer F.Cu) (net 14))
 (segment (start 163 71.625) (end 163 74.185002) (width 0.25) (layer F.Cu) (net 14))
 (segment (start 162.64499 71.26999) (end 163 71.625) (width 0.25) (layer F.Cu) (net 14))
 (segment (start 159.79999 69.659078) (end 161.410902 71.26999) (width 0.25) (layer F.Cu) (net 14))
 (segment (start 159.79999 69.000922) (end 159.79999 69.659078) (width 0.25) (layer F.Cu) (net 14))
 (segment (start 160.070922 68.72999) (end 159.79999 69.000922) (width 0.25) (layer F.Cu) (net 14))
 (segment (start 161.29501 68.72999) (end 160.070922 68.72999) (width 0.25) (layer F.Cu) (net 14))
 (segment (start 163 67.025) (end 161.29501 68.72999) (width 0.25) (layer F.Cu) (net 14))
 (segment (start 161.410902 71.26999) (end 162.64499 71.26999) (width 0.25) (layer F.Cu) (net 14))
 (segment (start 163 66.625) (end 163 67.025) (width 0.25) (layer F.Cu) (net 14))
 (segment (start 166.3 67.13) (end 165.325 67.13) (width 0.25) (layer F.Cu) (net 1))
 (segment (start 166.62501 67.45501) (end 166.3 67.13) (width 0.25) (layer F.Cu) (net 1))
 (segment (start 166.62501 73.52499) (end 166.62501 67.45501) (width 0.25) (layer F.Cu) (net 1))
 (segment (start 166.15 74) (end 166.62501 73.52499) (width 0.25) (layer F.Cu) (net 1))
 (segment (start 164.35 67.13) (end 165.325 67.13) (width 0.25) (layer F.Cu) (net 1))
 (segment (start 163.8 66.58) (end 164.35 67.13) (width 0.25) (layer F.Cu) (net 1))
 (segment (start 163.8 63.3) (end 163.8 66.58) (width 0.25) (layer F.Cu) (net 1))
 (segment (start 162.435 64.41) (end 163 64.975) (width 0.25) (layer F.Cu) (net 13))
 (segment (start 160.85 64.41) (end 162.435 64.41) (width 0.25) (layer F.Cu) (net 13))
 (segment (start 162.355 69.33) (end 163 69.975) (width 0.25) (layer F.Cu) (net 10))
 (segment (start 160.85 69.33) (end 162.355 69.33) (width 0.25) (layer F.Cu) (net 10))
 (via (at 168.6 68.4) (size 0.8) (drill 0.4) (layers F.Cu B.Cu) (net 5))
 (segment (start 170.275 68.4) (end 168.6 68.4) (width 0.25) (layer F.Cu) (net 5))
 (segment (start 167.399999 69.600001) (end 167.399999 71.399999) (width 0.25) (layer B.Cu) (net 5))
 (segment (start 168.6 68.4) (end 167.399999 69.600001) (width 0.25) (layer B.Cu) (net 5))
 (segment (start 169.4 72.4) (end 170 73) (width 0.25) (layer B.Cu) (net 5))
 (segment (start 168.4 72.4) (end 169.4 72.4) (width 0.25) (layer B.Cu) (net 5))
 (segment (start 167.399999 71.399999) (end 168.4 72.4) (width 0.25) (layer B.Cu) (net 5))
 (via (at 168.125 71) (size 0.8) (drill 0.4) (layers F.Cu B.Cu) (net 4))
 (segment (start 170 71) (end 168.125 71) (width 0.25) (layer B.Cu) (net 4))
 (segment (start 166.3 65.86) (end 165.325 65.86) (width 0.25) (layer F.Cu) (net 4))
 (segment (start 168.125 71) (end 167.4 71) (width 0.25) (layer F.Cu) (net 4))
 (segment (start 167.4 71) (end 167.1 70.7) (width 0.25) (layer F.Cu) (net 4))
 (segment (start 167.1 70.7) (end 167.1 66.66) (width 0.25) (layer F.Cu) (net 4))
 (segment (start 167.1 66.66) (end 166.3 65.86) (width 0.25) (layer F.Cu) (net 4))
 (via (at 167 64.6) (size 0.8) (drill 0.4) (layers F.Cu B.Cu) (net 3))
 (segment (start 166.99 64.59) (end 167 64.6) (width 0.25) (layer F.Cu) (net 3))
 (segment (start 165.325 64.59) (end 166.99 64.59) (width 0.25) (layer F.Cu) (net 3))
 (segment (start 167 65.3) (end 167 64.6) (width 0.25) (layer B.Cu) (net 3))
 (segment (start 170 68.55) (end 167 65.55) (width 0.25) (layer B.Cu) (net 3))
 (segment (start 167 65.55) (end 167 65.3) (width 0.25) (layer B.Cu) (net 3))
 (segment (start 170 69) (end 170 68.55) (width 0.25) (layer B.Cu) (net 3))
 (segment (start 168.6 65.29) (end 168.6 65.9) (width 0.25) (layer F.Cu) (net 2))
 (segment (start 169.3 64.59) (end 168.6 65.29) (width 0.25) (layer F.Cu) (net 2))
 (via (at 168.6 65.9) (size 0.8) (drill 0.4) (layers F.Cu B.Cu) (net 2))
 (segment (start 170.275 64.59) (end 169.3 64.59) (width 0.25) (layer F.Cu) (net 2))
 (segment (start 168.9 65.9) (end 170 67) (width 0.25) (layer B.Cu) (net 2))
 (segment (start 168.6 65.9) (end 168.9 65.9) (width 0.25) (layer B.Cu) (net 2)))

